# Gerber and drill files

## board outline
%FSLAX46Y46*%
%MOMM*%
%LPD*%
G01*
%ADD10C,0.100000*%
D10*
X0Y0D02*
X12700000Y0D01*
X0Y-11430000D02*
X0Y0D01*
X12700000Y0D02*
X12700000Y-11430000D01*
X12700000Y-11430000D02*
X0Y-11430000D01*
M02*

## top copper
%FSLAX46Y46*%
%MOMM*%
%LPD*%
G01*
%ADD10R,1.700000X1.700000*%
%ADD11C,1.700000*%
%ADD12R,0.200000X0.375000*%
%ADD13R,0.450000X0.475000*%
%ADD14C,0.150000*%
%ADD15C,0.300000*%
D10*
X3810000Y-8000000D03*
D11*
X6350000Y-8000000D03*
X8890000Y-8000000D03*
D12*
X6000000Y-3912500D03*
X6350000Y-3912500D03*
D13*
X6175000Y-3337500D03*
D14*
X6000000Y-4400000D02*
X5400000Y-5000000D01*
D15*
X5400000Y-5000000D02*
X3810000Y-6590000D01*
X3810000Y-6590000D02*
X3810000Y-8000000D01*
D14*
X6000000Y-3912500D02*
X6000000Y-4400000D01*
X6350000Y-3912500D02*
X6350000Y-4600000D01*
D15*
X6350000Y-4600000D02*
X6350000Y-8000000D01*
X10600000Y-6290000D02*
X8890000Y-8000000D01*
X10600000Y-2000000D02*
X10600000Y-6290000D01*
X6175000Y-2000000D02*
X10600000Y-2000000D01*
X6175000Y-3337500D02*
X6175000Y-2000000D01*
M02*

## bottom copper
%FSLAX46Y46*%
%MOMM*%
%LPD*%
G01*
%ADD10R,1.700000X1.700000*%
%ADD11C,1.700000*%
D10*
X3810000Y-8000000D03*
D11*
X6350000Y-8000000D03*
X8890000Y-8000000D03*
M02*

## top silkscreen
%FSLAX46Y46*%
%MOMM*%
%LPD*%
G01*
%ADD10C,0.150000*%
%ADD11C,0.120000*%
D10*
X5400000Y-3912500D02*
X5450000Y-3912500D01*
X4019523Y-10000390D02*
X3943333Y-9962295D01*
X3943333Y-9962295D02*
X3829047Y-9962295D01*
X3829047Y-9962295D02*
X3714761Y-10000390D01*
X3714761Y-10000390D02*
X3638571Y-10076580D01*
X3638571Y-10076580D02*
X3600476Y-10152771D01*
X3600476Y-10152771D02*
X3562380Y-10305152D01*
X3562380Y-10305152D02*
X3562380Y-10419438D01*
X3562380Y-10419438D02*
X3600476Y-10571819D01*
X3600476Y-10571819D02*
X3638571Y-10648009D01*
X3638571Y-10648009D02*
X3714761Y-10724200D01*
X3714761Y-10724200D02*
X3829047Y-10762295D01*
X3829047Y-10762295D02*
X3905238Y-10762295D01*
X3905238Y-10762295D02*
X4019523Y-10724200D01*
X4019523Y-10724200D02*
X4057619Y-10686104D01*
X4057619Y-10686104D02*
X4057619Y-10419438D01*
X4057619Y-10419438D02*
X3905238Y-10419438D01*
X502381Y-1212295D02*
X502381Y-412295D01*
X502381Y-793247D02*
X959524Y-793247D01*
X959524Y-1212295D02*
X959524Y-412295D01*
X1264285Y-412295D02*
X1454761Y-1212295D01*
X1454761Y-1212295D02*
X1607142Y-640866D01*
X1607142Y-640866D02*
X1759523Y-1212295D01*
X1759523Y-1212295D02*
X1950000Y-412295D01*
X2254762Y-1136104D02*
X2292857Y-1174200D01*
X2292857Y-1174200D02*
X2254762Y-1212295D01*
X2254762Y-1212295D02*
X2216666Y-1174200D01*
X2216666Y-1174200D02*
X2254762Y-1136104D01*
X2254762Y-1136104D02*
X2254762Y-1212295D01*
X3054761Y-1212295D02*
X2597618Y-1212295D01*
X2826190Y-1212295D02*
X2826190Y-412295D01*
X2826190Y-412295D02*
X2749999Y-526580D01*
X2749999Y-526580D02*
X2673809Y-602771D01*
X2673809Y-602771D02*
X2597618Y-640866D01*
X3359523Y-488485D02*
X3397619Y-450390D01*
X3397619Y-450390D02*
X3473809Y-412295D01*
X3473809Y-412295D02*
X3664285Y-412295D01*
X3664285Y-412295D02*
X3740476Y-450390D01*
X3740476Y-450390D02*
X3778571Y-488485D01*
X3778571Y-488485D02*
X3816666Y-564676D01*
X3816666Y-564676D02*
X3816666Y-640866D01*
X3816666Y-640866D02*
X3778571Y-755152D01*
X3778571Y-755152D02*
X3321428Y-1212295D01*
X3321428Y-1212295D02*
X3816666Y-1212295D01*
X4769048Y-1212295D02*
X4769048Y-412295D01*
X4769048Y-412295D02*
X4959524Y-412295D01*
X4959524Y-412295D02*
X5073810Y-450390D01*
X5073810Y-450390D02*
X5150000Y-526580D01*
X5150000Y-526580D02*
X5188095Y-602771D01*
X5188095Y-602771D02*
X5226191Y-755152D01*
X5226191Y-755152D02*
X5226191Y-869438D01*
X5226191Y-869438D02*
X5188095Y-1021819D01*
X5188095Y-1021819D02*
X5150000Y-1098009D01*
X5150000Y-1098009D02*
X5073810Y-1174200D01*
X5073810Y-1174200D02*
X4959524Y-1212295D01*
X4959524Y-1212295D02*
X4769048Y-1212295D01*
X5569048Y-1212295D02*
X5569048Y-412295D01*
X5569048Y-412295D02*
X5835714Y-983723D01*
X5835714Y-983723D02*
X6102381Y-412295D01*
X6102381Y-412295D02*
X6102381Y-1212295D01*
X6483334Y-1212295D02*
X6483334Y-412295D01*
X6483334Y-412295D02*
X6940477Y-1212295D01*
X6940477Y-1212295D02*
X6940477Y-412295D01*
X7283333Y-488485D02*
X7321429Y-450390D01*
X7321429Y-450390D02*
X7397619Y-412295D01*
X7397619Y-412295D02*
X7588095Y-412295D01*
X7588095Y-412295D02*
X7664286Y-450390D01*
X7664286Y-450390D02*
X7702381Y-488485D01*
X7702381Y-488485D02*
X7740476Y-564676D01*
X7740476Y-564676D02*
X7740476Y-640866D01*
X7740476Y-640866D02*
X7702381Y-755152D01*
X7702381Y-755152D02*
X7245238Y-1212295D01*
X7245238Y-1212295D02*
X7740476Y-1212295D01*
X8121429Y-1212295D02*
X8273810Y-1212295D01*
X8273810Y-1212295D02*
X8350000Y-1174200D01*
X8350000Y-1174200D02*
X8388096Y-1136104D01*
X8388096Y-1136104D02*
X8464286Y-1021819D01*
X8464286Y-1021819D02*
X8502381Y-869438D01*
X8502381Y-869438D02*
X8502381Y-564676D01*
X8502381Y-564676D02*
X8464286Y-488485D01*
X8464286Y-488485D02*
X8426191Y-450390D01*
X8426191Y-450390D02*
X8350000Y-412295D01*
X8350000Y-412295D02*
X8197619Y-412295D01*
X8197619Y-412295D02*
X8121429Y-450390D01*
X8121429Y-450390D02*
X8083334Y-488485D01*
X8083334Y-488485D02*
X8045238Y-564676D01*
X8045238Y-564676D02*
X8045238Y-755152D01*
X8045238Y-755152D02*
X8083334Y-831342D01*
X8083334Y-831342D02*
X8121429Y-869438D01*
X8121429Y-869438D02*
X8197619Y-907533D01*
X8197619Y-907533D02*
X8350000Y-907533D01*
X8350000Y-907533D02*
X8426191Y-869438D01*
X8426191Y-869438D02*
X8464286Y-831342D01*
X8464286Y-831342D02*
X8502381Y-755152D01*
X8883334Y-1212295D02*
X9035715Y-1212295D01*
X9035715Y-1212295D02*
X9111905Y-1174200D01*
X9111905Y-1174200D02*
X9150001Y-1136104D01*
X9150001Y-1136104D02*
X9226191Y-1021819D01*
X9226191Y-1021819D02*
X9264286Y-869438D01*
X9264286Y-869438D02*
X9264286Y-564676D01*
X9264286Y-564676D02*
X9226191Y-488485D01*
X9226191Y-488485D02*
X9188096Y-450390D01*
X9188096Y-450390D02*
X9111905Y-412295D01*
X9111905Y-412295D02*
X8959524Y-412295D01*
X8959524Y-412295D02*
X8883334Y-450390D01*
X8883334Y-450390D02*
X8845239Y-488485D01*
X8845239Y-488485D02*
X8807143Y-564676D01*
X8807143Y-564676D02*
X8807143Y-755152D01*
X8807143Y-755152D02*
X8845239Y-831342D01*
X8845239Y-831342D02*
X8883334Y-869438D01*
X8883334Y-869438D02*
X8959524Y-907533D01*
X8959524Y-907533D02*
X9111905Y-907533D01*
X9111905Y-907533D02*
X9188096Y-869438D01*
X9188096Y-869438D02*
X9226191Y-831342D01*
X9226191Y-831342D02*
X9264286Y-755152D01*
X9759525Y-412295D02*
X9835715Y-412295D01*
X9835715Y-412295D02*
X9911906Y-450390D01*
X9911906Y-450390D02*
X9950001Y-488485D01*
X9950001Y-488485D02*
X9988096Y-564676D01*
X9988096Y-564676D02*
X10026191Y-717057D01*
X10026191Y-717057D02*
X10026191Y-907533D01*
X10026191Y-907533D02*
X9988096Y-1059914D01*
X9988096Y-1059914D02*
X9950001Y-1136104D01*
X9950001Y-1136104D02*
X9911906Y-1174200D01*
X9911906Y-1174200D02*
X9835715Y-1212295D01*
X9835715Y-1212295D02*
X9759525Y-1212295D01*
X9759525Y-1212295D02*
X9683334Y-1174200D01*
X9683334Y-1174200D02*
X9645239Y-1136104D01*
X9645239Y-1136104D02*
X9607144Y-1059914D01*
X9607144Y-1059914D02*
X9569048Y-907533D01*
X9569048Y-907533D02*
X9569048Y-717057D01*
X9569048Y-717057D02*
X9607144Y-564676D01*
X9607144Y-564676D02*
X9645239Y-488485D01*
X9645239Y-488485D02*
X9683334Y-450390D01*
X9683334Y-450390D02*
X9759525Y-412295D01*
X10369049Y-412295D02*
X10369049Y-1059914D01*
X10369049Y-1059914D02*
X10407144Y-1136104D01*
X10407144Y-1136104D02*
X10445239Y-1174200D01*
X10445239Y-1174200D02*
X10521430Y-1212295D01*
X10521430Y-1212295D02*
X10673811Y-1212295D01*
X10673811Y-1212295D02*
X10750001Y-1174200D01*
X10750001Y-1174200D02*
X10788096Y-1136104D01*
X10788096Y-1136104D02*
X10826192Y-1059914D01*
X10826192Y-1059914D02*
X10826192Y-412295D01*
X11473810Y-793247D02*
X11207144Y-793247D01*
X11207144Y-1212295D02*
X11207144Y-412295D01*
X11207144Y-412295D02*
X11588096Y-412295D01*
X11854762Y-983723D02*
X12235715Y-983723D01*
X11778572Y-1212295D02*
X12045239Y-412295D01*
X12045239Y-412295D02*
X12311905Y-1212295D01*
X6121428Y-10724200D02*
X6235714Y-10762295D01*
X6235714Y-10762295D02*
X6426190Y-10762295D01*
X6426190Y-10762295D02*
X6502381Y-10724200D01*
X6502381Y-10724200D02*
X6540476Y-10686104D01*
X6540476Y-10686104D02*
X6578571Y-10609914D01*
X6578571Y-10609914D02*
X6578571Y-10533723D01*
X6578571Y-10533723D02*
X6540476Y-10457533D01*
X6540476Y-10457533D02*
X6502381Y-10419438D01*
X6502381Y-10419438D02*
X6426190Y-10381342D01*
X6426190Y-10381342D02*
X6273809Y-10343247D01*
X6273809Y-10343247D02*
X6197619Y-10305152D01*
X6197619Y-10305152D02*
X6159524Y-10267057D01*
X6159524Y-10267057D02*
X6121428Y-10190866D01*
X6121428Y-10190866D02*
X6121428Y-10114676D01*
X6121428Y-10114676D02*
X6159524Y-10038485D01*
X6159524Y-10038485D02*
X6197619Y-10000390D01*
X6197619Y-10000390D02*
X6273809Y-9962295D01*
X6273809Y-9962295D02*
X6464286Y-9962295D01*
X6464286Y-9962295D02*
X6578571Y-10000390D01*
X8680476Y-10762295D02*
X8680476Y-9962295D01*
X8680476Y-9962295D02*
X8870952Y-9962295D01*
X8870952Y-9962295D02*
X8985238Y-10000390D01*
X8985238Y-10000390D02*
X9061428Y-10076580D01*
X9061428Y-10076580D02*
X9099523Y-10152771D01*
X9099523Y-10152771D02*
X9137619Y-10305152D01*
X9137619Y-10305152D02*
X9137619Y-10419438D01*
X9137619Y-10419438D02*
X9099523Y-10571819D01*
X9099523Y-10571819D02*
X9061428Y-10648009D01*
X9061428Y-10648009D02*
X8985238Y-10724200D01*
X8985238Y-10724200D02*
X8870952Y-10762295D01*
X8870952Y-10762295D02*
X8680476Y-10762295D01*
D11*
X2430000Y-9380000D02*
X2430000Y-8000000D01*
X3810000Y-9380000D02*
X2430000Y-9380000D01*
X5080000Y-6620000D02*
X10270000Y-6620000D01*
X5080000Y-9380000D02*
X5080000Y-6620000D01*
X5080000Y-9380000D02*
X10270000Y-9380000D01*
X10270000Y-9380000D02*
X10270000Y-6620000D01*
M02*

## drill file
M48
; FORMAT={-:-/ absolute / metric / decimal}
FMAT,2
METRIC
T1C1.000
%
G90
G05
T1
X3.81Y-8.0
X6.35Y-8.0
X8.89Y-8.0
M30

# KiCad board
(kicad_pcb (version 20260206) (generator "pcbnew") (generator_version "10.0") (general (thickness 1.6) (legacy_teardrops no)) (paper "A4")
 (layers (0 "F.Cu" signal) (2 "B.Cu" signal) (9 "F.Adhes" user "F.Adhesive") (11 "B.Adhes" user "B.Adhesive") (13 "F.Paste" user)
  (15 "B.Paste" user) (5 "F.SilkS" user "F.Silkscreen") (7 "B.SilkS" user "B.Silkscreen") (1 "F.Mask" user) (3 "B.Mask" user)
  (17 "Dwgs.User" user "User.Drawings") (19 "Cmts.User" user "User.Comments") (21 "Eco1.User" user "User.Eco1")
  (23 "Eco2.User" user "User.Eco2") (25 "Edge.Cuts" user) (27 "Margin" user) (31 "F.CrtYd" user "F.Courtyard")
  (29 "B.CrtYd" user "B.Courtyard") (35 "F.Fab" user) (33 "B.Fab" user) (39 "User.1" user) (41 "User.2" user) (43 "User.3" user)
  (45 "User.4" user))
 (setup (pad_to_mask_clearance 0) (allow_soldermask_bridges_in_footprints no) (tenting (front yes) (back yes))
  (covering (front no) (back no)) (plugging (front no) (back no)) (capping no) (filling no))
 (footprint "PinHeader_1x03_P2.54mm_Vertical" (layer "F.Cu") (at 3.81 8 90)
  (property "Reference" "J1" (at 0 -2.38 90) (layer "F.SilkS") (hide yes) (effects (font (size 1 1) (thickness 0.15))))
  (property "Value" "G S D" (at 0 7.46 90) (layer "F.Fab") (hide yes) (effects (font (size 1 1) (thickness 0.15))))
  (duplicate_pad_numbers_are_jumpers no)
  (fp_line (start -1.38 -1.38) (end 0 -1.38) (stroke (width 0.12) (type solid)) (layer "F.SilkS"))
  (fp_line (start -1.38 0) (end -1.38 -1.38) (stroke (width 0.12) (type solid)) (layer "F.SilkS"))
  (fp_line (start 1.38 1.27) (end 1.38 6.46) (stroke (width 0.12) (type solid)) (layer "F.SilkS"))
  (fp_line (start -1.38 1.27) (end 1.38 1.27) (stroke (width 0.12) (type solid)) (layer "F.SilkS"))
  (fp_line (start -1.38 1.27) (end -1.38 6.46) (stroke (width 0.12) (type solid)) (layer "F.SilkS"))
  (fp_line (start -1.38 6.46) (end 1.38 6.46) (stroke (width 0.12) (type solid)) (layer "F.SilkS"))
  (pad "1" thru_hole rect (at 0 0 90) (size 1.7 1.7) (drill 1) (layers "*.Cu" "*.Mask") (remove_unused_layers no) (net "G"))
  (pad "2" thru_hole circle (at 0 2.54 90) (size 1.7 1.7) (drill 1) (layers "*.Cu" "*.Mask") (remove_unused_layers no) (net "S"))
  (pad "3" thru_hole circle (at 0 5.08 90) (size 1.7 1.7) (drill 1) (layers "*.Cu" "*.Mask") (remove_unused_layers no) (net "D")))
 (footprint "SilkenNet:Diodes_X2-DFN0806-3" (layer "F.Cu") (at 6.175 3.6)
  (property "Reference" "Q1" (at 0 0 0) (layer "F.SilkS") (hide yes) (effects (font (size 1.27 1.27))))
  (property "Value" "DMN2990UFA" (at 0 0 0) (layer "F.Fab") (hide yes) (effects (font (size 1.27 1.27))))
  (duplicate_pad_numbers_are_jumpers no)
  (pad "1" smd rect (at -0.175 0.3125) (size 0.2 0.375) (layers "F.Cu" "F.Mask" "F.Paste") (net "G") (thermal_bridge_angle 45))
  (pad "2" smd rect (at 0.175 0.3125) (size 0.2 0.375) (layers "F.Cu" "F.Mask" "F.Paste") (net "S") (thermal_bridge_angle 45))
  (pad "3" smd rect (at 0 -0.2625) (size 0.45 0.475) (layers "F.Cu" "F.Mask" "F.Paste") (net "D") (thermal_bridge_angle 45)))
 (gr_line (start 5.4 3.9125) (end 5.45 3.9125) (stroke (width 0.15) (type default)) (layer "F.SilkS"))
 (gr_line (start 0 0) (end 12.7 0) (stroke (width 0.1) (type default)) (layer "Edge.Cuts"))
 (gr_line (start 0 11.43) (end 0 0) (stroke (width 0.1) (type default)) (layer "Edge.Cuts"))
 (gr_line (start 12.7 0) (end 12.7 11.43) (stroke (width 0.1) (type default)) (layer "Edge.Cuts"))
 (gr_line (start 12.7 11.43) (end 0 11.43) (stroke (width 0.1) (type default)) (layer "Edge.Cuts"))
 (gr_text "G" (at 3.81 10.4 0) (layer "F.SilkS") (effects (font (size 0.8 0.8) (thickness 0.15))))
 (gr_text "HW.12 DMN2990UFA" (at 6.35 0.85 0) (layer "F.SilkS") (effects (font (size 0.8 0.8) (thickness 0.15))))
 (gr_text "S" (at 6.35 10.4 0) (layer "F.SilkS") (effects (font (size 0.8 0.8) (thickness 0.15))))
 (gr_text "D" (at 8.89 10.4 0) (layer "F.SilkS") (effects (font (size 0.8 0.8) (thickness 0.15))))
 (segment (start 6 4.4) (end 5.4 5) (width 0.15) (layer "F.Cu") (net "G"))
 (segment (start 5.4 5) (end 3.81 6.59) (width 0.3) (layer "F.Cu") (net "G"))
 (segment (start 3.81 6.59) (end 3.81 8) (width 0.3) (layer "F.Cu") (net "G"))
 (segment (start 6 3.9125) (end 6 4.4) (width 0.15) (layer "F.Cu") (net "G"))
 (segment (start 6.35 3.9125) (end 6.35 4.6) (width 0.15) (layer "F.Cu") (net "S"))
 (segment (start 6.35 4.6) (end 6.35 8) (width 0.3) (layer "F.Cu") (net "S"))
 (segment (start 10.6 6.29) (end 8.89 8) (width 0.3) (layer "F.Cu") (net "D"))
 (segment (start 10.6 2) (end 10.6 6.29) (width 0.3) (layer "F.Cu") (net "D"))
 (segment (start 6.175 2) (end 10.6 2) (width 0.3) (layer "F.Cu") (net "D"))
 (segment (start 6.175 3.3375) (end 6.175 2) (width 0.3) (layer "F.Cu") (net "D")))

